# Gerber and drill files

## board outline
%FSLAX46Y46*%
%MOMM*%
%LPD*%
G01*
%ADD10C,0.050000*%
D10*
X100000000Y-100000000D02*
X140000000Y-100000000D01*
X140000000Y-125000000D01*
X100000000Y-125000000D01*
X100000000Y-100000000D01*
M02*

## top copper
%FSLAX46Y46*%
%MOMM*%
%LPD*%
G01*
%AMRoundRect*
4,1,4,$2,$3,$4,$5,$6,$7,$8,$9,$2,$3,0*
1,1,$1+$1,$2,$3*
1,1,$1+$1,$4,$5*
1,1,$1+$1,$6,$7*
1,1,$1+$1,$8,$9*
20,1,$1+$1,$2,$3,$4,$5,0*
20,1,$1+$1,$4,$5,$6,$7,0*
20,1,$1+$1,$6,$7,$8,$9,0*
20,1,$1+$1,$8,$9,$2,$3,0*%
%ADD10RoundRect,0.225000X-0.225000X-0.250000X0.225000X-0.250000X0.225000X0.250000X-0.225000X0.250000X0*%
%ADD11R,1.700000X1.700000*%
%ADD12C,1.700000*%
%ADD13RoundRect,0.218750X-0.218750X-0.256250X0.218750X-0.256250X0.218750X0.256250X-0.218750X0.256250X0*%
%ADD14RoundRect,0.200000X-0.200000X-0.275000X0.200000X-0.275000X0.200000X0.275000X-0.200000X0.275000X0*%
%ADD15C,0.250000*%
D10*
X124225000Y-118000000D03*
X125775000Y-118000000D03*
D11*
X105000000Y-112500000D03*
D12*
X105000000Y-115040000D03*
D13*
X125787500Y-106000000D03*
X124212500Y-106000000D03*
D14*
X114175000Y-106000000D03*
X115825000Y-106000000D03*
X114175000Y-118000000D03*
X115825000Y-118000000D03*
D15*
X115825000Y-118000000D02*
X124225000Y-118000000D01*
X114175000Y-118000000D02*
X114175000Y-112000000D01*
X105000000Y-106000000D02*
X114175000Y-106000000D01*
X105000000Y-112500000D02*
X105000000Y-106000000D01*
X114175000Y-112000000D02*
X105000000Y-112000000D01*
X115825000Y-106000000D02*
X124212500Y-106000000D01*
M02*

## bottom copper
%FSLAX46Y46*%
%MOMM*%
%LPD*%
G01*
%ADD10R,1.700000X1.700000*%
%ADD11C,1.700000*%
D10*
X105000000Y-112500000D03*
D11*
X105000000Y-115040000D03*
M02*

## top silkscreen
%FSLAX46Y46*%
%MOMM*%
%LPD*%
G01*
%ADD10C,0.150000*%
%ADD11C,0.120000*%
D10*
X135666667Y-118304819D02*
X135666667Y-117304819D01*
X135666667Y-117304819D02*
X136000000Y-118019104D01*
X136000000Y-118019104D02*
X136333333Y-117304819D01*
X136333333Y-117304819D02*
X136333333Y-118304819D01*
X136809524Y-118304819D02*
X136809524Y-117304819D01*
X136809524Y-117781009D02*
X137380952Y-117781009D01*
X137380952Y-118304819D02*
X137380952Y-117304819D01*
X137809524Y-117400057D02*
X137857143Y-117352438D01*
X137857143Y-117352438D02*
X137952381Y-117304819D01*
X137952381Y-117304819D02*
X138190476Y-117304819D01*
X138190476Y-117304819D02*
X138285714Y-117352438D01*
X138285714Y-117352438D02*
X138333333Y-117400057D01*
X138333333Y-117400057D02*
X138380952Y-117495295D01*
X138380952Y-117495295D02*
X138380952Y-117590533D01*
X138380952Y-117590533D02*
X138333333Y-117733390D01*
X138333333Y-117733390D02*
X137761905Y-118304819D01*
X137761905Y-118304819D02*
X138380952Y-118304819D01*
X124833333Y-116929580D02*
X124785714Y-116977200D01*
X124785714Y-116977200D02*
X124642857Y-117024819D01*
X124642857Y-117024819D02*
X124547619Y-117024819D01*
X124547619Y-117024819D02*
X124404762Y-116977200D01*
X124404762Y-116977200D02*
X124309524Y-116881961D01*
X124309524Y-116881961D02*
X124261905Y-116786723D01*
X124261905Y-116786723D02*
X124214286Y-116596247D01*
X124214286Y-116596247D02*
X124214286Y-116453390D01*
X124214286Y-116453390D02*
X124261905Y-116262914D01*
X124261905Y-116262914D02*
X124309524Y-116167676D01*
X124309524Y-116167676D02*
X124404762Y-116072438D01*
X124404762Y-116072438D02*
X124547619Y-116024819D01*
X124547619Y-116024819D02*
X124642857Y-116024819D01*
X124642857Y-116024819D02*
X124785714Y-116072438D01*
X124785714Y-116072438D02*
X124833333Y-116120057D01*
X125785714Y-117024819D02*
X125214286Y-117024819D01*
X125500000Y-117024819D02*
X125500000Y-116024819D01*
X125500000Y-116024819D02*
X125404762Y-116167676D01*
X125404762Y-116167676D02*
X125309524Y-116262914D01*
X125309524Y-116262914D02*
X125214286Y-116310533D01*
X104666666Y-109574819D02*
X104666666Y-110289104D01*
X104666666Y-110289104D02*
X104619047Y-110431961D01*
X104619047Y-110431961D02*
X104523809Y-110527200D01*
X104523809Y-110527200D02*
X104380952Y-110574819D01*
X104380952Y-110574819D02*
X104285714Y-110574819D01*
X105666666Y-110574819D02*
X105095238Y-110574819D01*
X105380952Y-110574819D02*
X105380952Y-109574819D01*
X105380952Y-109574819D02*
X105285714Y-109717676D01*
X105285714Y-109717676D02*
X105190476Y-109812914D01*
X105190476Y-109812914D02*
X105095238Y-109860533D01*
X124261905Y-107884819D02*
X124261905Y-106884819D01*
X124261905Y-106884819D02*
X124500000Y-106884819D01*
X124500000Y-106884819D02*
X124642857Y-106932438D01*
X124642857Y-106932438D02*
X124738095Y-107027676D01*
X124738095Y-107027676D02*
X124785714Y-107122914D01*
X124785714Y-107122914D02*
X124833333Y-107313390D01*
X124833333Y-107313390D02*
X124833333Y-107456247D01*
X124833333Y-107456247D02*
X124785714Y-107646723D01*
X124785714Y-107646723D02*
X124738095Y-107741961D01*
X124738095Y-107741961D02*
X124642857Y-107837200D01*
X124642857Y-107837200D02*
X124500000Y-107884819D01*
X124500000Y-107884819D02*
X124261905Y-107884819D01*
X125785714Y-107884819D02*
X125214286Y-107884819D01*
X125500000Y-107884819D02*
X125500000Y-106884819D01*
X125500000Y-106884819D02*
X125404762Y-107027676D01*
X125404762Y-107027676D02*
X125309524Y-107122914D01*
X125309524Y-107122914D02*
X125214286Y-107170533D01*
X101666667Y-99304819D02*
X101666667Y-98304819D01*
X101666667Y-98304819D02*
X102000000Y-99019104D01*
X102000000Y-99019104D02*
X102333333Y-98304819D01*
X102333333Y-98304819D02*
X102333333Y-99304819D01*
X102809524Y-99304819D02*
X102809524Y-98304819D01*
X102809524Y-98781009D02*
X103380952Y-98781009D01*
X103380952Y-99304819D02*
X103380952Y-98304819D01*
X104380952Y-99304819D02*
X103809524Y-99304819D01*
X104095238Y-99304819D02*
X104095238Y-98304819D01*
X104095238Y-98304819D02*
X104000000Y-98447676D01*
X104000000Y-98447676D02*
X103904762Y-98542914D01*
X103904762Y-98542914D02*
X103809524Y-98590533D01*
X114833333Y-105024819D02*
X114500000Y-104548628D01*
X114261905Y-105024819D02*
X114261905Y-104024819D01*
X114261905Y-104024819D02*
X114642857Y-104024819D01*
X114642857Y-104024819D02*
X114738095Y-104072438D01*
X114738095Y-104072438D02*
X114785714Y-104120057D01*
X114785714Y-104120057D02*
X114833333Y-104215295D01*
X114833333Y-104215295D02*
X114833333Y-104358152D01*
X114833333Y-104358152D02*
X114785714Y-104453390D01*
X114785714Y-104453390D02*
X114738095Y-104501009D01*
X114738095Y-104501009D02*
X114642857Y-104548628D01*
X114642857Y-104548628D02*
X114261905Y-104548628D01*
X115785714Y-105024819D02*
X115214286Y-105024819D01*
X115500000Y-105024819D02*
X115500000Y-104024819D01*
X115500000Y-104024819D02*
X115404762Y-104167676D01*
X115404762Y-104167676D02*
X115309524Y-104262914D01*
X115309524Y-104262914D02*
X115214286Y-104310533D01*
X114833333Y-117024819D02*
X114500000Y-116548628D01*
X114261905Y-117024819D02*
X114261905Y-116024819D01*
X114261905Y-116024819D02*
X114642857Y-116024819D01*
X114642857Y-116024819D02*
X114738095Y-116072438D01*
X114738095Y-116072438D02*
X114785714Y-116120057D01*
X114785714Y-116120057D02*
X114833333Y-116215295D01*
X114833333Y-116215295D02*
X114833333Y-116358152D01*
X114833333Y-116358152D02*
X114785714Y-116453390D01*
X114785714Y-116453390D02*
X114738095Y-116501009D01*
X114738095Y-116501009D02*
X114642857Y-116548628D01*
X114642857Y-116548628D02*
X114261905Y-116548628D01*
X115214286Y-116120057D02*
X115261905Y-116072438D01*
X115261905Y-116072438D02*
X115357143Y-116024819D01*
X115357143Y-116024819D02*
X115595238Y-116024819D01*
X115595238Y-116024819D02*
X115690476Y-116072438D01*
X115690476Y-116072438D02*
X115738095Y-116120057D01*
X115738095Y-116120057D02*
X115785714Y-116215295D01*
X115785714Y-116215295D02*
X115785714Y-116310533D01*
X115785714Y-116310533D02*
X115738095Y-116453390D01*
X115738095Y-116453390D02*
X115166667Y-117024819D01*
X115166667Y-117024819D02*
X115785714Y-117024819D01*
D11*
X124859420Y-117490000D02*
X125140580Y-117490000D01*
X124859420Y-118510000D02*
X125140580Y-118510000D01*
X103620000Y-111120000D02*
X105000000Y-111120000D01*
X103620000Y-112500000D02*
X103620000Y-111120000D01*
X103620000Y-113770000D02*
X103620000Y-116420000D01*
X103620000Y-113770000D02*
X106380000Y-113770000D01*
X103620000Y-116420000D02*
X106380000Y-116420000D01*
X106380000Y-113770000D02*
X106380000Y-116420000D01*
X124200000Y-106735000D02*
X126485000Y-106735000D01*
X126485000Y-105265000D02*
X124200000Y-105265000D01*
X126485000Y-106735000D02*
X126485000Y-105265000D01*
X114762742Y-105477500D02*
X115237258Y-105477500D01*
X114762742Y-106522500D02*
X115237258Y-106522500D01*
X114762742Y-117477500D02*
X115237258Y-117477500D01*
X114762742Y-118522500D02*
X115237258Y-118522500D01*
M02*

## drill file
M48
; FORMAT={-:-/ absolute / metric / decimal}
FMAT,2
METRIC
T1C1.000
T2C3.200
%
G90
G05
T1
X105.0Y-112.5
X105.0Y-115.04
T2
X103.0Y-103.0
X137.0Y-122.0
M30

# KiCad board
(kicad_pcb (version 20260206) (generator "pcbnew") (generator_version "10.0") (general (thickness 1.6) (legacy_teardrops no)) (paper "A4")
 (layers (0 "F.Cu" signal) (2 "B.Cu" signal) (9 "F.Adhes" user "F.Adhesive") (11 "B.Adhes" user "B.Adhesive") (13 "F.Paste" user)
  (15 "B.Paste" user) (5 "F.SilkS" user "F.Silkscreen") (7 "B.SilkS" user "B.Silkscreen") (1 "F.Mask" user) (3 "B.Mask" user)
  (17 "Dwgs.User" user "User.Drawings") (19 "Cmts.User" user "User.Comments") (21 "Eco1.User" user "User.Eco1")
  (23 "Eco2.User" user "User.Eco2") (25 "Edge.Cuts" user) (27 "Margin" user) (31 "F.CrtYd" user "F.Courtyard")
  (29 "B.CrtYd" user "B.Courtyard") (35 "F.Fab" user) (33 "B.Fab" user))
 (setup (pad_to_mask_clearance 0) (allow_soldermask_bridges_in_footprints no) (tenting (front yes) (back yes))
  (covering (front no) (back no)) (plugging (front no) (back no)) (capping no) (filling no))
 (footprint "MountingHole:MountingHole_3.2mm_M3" (layer "F.Cu") (at 137 122)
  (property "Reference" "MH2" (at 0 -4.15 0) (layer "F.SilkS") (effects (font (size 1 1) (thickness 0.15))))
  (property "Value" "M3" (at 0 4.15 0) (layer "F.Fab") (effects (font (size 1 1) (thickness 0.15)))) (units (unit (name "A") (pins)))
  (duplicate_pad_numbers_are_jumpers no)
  (pad "" np_thru_hole circle (at 0 0) (size 3.2 3.2) (drill 3.2) (layers "*.Cu" "*.Mask")))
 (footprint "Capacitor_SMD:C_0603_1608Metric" (layer "F.Cu") (at 125 118)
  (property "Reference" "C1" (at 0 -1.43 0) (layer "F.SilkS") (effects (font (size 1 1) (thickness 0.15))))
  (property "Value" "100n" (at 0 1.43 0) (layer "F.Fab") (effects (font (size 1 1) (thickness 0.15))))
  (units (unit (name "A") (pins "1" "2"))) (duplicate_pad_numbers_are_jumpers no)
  (fp_line (start -0.14058 -0.51) (end 0.14058 -0.51) (stroke (width 0.12) (type solid)) (layer "F.SilkS"))
  (fp_line (start -0.14058 0.51) (end 0.14058 0.51) (stroke (width 0.12) (type solid)) (layer "F.SilkS"))
  (pad "1" smd roundrect (at -0.775 0) (size 0.9 0.95) (layers "F.Cu" "F.Mask" "F.Paste") (roundrect_rratio 0.25) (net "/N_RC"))
  (pad "2" smd roundrect (at 0.775 0) (size 0.9 0.95) (layers "F.Cu" "F.Mask" "F.Paste") (roundrect_rratio 0.25) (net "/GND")))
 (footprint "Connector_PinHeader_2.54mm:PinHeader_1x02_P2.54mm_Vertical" (layer "F.Cu") (at 105 112.5)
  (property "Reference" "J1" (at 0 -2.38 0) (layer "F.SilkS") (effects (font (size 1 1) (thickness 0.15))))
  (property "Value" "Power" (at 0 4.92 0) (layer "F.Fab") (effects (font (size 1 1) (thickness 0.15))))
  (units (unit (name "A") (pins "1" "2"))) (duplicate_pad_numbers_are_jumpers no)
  (fp_line (start -1.38 -1.38) (end 0 -1.38) (stroke (width 0.12) (type solid)) (layer "F.SilkS"))
  (fp_line (start -1.38 0) (end -1.38 -1.38) (stroke (width 0.12) (type solid)) (layer "F.SilkS"))
  (fp_line (start -1.38 1.27) (end -1.38 3.92) (stroke (width 0.12) (type solid)) (layer "F.SilkS"))
  (fp_line (start -1.38 1.27) (end 1.38 1.27) (stroke (width 0.12) (type solid)) (layer "F.SilkS"))
  (fp_line (start -1.38 3.92) (end 1.38 3.92) (stroke (width 0.12) (type solid)) (layer "F.SilkS"))
  (fp_line (start 1.38 1.27) (end 1.38 3.92) (stroke (width 0.12) (type solid)) (layer "F.SilkS"))
  (pad "1" thru_hole rect (at 0 0) (size 1.7 1.7) (drill 1) (layers "*.Cu" "*.Mask") (remove_unused_layers no) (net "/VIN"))
  (pad "2" thru_hole circle (at 0 2.54) (size 1.7 1.7) (drill 1) (layers "*.Cu" "*.Mask") (remove_unused_layers no) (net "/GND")))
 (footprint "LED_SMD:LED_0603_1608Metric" (layer "F.Cu") (at 125 106 180)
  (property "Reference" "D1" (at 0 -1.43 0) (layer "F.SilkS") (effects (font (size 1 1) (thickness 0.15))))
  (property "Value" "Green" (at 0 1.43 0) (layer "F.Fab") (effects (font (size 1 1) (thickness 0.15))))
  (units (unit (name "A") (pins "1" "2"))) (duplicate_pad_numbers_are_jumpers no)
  (fp_line (start 0.8 -0.735) (end -1.485 -0.735) (stroke (width 0.12) (type solid)) (layer "F.SilkS"))
  (fp_line (start -1.485 0.735) (end 0.8 0.735) (stroke (width 0.12) (type solid)) (layer "F.SilkS"))
  (fp_line (start -1.485 -0.735) (end -1.485 0.735) (stroke (width 0.12) (type solid)) (layer "F.SilkS"))
  (pad "1" smd roundrect (at -0.7875 0) (size 0.875 0.95) (layers "F.Cu" "F.Mask" "F.Paste") (roundrect_rratio 0.25) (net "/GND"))
  (pad "2" smd roundrect (at 0.7875 0) (size 0.875 0.95) (layers "F.Cu" "F.Mask" "F.Paste") (roundrect_rratio 0.25) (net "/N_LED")))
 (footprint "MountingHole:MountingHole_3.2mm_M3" (layer "F.Cu") (at 103 103)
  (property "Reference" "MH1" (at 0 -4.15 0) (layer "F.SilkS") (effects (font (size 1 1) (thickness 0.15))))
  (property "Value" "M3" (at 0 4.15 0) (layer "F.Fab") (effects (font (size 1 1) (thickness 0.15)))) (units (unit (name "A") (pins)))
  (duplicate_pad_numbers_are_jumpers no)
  (pad "" np_thru_hole circle (at 0 0) (size 3.2 3.2) (drill 3.2) (layers "*.Cu" "*.Mask")))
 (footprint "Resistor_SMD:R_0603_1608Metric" (layer "F.Cu") (at 115 106)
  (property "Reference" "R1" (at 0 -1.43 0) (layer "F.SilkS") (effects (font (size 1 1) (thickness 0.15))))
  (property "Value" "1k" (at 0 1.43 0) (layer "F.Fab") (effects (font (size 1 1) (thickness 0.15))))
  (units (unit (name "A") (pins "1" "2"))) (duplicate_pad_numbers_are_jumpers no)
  (fp_line (start -0.237258 -0.5225) (end 0.237258 -0.5225) (stroke (width 0.12) (type solid)) (layer "F.SilkS"))
  (fp_line (start -0.237258 0.5225) (end 0.237258 0.5225) (stroke (width 0.12) (type solid)) (layer "F.SilkS"))
  (pad "1" smd roundrect (at -0.825 0) (size 0.8 0.95) (layers "F.Cu" "F.Mask" "F.Paste") (roundrect_rratio 0.25) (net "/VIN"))
  (pad "2" smd roundrect (at 0.825 0) (size 0.8 0.95) (layers "F.Cu" "F.Mask" "F.Paste") (roundrect_rratio 0.25) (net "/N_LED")))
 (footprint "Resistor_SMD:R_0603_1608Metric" (layer "F.Cu") (at 115 118)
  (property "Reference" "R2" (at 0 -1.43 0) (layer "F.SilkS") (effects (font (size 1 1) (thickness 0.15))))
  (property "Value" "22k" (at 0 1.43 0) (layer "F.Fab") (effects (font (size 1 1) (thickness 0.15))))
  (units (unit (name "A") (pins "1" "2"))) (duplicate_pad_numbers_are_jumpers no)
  (fp_line (start -0.237258 -0.5225) (end 0.237258 -0.5225) (stroke (width 0.12) (type solid)) (layer "F.SilkS"))
  (fp_line (start -0.237258 0.5225) (end 0.237258 0.5225) (stroke (width 0.12) (type solid)) (layer "F.SilkS"))
  (pad "1" smd roundrect (at -0.825 0) (size 0.8 0.95) (layers "F.Cu" "F.Mask" "F.Paste") (roundrect_rratio 0.25) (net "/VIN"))
  (pad "2" smd roundrect (at 0.825 0) (size 0.8 0.95) (layers "F.Cu" "F.Mask" "F.Paste") (roundrect_rratio 0.25) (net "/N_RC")))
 (gr_rect (start 100 100) (end 140 125) (stroke (width 0.05) (type default)) (fill no) (layer "Edge.Cuts"))
 (segment (start 115.825 118) (end 124.225 118) (width 0.25) (layer "F.Cu") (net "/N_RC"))
 (segment (start 114.175 118) (end 114.175 112) (width 0.25) (layer "F.Cu") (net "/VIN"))
 (segment (start 105 106) (end 114.175 106) (width 0.25) (layer "F.Cu") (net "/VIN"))
 (segment (start 105 112.5) (end 105 106) (width 0.25) (layer "F.Cu") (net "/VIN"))
 (segment (start 114.175 112) (end 105 112) (width 0.25) (layer "F.Cu") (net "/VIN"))
 (segment (start 115.825 106) (end 124.2125 106) (width 0.25) (layer "F.Cu") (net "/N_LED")))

